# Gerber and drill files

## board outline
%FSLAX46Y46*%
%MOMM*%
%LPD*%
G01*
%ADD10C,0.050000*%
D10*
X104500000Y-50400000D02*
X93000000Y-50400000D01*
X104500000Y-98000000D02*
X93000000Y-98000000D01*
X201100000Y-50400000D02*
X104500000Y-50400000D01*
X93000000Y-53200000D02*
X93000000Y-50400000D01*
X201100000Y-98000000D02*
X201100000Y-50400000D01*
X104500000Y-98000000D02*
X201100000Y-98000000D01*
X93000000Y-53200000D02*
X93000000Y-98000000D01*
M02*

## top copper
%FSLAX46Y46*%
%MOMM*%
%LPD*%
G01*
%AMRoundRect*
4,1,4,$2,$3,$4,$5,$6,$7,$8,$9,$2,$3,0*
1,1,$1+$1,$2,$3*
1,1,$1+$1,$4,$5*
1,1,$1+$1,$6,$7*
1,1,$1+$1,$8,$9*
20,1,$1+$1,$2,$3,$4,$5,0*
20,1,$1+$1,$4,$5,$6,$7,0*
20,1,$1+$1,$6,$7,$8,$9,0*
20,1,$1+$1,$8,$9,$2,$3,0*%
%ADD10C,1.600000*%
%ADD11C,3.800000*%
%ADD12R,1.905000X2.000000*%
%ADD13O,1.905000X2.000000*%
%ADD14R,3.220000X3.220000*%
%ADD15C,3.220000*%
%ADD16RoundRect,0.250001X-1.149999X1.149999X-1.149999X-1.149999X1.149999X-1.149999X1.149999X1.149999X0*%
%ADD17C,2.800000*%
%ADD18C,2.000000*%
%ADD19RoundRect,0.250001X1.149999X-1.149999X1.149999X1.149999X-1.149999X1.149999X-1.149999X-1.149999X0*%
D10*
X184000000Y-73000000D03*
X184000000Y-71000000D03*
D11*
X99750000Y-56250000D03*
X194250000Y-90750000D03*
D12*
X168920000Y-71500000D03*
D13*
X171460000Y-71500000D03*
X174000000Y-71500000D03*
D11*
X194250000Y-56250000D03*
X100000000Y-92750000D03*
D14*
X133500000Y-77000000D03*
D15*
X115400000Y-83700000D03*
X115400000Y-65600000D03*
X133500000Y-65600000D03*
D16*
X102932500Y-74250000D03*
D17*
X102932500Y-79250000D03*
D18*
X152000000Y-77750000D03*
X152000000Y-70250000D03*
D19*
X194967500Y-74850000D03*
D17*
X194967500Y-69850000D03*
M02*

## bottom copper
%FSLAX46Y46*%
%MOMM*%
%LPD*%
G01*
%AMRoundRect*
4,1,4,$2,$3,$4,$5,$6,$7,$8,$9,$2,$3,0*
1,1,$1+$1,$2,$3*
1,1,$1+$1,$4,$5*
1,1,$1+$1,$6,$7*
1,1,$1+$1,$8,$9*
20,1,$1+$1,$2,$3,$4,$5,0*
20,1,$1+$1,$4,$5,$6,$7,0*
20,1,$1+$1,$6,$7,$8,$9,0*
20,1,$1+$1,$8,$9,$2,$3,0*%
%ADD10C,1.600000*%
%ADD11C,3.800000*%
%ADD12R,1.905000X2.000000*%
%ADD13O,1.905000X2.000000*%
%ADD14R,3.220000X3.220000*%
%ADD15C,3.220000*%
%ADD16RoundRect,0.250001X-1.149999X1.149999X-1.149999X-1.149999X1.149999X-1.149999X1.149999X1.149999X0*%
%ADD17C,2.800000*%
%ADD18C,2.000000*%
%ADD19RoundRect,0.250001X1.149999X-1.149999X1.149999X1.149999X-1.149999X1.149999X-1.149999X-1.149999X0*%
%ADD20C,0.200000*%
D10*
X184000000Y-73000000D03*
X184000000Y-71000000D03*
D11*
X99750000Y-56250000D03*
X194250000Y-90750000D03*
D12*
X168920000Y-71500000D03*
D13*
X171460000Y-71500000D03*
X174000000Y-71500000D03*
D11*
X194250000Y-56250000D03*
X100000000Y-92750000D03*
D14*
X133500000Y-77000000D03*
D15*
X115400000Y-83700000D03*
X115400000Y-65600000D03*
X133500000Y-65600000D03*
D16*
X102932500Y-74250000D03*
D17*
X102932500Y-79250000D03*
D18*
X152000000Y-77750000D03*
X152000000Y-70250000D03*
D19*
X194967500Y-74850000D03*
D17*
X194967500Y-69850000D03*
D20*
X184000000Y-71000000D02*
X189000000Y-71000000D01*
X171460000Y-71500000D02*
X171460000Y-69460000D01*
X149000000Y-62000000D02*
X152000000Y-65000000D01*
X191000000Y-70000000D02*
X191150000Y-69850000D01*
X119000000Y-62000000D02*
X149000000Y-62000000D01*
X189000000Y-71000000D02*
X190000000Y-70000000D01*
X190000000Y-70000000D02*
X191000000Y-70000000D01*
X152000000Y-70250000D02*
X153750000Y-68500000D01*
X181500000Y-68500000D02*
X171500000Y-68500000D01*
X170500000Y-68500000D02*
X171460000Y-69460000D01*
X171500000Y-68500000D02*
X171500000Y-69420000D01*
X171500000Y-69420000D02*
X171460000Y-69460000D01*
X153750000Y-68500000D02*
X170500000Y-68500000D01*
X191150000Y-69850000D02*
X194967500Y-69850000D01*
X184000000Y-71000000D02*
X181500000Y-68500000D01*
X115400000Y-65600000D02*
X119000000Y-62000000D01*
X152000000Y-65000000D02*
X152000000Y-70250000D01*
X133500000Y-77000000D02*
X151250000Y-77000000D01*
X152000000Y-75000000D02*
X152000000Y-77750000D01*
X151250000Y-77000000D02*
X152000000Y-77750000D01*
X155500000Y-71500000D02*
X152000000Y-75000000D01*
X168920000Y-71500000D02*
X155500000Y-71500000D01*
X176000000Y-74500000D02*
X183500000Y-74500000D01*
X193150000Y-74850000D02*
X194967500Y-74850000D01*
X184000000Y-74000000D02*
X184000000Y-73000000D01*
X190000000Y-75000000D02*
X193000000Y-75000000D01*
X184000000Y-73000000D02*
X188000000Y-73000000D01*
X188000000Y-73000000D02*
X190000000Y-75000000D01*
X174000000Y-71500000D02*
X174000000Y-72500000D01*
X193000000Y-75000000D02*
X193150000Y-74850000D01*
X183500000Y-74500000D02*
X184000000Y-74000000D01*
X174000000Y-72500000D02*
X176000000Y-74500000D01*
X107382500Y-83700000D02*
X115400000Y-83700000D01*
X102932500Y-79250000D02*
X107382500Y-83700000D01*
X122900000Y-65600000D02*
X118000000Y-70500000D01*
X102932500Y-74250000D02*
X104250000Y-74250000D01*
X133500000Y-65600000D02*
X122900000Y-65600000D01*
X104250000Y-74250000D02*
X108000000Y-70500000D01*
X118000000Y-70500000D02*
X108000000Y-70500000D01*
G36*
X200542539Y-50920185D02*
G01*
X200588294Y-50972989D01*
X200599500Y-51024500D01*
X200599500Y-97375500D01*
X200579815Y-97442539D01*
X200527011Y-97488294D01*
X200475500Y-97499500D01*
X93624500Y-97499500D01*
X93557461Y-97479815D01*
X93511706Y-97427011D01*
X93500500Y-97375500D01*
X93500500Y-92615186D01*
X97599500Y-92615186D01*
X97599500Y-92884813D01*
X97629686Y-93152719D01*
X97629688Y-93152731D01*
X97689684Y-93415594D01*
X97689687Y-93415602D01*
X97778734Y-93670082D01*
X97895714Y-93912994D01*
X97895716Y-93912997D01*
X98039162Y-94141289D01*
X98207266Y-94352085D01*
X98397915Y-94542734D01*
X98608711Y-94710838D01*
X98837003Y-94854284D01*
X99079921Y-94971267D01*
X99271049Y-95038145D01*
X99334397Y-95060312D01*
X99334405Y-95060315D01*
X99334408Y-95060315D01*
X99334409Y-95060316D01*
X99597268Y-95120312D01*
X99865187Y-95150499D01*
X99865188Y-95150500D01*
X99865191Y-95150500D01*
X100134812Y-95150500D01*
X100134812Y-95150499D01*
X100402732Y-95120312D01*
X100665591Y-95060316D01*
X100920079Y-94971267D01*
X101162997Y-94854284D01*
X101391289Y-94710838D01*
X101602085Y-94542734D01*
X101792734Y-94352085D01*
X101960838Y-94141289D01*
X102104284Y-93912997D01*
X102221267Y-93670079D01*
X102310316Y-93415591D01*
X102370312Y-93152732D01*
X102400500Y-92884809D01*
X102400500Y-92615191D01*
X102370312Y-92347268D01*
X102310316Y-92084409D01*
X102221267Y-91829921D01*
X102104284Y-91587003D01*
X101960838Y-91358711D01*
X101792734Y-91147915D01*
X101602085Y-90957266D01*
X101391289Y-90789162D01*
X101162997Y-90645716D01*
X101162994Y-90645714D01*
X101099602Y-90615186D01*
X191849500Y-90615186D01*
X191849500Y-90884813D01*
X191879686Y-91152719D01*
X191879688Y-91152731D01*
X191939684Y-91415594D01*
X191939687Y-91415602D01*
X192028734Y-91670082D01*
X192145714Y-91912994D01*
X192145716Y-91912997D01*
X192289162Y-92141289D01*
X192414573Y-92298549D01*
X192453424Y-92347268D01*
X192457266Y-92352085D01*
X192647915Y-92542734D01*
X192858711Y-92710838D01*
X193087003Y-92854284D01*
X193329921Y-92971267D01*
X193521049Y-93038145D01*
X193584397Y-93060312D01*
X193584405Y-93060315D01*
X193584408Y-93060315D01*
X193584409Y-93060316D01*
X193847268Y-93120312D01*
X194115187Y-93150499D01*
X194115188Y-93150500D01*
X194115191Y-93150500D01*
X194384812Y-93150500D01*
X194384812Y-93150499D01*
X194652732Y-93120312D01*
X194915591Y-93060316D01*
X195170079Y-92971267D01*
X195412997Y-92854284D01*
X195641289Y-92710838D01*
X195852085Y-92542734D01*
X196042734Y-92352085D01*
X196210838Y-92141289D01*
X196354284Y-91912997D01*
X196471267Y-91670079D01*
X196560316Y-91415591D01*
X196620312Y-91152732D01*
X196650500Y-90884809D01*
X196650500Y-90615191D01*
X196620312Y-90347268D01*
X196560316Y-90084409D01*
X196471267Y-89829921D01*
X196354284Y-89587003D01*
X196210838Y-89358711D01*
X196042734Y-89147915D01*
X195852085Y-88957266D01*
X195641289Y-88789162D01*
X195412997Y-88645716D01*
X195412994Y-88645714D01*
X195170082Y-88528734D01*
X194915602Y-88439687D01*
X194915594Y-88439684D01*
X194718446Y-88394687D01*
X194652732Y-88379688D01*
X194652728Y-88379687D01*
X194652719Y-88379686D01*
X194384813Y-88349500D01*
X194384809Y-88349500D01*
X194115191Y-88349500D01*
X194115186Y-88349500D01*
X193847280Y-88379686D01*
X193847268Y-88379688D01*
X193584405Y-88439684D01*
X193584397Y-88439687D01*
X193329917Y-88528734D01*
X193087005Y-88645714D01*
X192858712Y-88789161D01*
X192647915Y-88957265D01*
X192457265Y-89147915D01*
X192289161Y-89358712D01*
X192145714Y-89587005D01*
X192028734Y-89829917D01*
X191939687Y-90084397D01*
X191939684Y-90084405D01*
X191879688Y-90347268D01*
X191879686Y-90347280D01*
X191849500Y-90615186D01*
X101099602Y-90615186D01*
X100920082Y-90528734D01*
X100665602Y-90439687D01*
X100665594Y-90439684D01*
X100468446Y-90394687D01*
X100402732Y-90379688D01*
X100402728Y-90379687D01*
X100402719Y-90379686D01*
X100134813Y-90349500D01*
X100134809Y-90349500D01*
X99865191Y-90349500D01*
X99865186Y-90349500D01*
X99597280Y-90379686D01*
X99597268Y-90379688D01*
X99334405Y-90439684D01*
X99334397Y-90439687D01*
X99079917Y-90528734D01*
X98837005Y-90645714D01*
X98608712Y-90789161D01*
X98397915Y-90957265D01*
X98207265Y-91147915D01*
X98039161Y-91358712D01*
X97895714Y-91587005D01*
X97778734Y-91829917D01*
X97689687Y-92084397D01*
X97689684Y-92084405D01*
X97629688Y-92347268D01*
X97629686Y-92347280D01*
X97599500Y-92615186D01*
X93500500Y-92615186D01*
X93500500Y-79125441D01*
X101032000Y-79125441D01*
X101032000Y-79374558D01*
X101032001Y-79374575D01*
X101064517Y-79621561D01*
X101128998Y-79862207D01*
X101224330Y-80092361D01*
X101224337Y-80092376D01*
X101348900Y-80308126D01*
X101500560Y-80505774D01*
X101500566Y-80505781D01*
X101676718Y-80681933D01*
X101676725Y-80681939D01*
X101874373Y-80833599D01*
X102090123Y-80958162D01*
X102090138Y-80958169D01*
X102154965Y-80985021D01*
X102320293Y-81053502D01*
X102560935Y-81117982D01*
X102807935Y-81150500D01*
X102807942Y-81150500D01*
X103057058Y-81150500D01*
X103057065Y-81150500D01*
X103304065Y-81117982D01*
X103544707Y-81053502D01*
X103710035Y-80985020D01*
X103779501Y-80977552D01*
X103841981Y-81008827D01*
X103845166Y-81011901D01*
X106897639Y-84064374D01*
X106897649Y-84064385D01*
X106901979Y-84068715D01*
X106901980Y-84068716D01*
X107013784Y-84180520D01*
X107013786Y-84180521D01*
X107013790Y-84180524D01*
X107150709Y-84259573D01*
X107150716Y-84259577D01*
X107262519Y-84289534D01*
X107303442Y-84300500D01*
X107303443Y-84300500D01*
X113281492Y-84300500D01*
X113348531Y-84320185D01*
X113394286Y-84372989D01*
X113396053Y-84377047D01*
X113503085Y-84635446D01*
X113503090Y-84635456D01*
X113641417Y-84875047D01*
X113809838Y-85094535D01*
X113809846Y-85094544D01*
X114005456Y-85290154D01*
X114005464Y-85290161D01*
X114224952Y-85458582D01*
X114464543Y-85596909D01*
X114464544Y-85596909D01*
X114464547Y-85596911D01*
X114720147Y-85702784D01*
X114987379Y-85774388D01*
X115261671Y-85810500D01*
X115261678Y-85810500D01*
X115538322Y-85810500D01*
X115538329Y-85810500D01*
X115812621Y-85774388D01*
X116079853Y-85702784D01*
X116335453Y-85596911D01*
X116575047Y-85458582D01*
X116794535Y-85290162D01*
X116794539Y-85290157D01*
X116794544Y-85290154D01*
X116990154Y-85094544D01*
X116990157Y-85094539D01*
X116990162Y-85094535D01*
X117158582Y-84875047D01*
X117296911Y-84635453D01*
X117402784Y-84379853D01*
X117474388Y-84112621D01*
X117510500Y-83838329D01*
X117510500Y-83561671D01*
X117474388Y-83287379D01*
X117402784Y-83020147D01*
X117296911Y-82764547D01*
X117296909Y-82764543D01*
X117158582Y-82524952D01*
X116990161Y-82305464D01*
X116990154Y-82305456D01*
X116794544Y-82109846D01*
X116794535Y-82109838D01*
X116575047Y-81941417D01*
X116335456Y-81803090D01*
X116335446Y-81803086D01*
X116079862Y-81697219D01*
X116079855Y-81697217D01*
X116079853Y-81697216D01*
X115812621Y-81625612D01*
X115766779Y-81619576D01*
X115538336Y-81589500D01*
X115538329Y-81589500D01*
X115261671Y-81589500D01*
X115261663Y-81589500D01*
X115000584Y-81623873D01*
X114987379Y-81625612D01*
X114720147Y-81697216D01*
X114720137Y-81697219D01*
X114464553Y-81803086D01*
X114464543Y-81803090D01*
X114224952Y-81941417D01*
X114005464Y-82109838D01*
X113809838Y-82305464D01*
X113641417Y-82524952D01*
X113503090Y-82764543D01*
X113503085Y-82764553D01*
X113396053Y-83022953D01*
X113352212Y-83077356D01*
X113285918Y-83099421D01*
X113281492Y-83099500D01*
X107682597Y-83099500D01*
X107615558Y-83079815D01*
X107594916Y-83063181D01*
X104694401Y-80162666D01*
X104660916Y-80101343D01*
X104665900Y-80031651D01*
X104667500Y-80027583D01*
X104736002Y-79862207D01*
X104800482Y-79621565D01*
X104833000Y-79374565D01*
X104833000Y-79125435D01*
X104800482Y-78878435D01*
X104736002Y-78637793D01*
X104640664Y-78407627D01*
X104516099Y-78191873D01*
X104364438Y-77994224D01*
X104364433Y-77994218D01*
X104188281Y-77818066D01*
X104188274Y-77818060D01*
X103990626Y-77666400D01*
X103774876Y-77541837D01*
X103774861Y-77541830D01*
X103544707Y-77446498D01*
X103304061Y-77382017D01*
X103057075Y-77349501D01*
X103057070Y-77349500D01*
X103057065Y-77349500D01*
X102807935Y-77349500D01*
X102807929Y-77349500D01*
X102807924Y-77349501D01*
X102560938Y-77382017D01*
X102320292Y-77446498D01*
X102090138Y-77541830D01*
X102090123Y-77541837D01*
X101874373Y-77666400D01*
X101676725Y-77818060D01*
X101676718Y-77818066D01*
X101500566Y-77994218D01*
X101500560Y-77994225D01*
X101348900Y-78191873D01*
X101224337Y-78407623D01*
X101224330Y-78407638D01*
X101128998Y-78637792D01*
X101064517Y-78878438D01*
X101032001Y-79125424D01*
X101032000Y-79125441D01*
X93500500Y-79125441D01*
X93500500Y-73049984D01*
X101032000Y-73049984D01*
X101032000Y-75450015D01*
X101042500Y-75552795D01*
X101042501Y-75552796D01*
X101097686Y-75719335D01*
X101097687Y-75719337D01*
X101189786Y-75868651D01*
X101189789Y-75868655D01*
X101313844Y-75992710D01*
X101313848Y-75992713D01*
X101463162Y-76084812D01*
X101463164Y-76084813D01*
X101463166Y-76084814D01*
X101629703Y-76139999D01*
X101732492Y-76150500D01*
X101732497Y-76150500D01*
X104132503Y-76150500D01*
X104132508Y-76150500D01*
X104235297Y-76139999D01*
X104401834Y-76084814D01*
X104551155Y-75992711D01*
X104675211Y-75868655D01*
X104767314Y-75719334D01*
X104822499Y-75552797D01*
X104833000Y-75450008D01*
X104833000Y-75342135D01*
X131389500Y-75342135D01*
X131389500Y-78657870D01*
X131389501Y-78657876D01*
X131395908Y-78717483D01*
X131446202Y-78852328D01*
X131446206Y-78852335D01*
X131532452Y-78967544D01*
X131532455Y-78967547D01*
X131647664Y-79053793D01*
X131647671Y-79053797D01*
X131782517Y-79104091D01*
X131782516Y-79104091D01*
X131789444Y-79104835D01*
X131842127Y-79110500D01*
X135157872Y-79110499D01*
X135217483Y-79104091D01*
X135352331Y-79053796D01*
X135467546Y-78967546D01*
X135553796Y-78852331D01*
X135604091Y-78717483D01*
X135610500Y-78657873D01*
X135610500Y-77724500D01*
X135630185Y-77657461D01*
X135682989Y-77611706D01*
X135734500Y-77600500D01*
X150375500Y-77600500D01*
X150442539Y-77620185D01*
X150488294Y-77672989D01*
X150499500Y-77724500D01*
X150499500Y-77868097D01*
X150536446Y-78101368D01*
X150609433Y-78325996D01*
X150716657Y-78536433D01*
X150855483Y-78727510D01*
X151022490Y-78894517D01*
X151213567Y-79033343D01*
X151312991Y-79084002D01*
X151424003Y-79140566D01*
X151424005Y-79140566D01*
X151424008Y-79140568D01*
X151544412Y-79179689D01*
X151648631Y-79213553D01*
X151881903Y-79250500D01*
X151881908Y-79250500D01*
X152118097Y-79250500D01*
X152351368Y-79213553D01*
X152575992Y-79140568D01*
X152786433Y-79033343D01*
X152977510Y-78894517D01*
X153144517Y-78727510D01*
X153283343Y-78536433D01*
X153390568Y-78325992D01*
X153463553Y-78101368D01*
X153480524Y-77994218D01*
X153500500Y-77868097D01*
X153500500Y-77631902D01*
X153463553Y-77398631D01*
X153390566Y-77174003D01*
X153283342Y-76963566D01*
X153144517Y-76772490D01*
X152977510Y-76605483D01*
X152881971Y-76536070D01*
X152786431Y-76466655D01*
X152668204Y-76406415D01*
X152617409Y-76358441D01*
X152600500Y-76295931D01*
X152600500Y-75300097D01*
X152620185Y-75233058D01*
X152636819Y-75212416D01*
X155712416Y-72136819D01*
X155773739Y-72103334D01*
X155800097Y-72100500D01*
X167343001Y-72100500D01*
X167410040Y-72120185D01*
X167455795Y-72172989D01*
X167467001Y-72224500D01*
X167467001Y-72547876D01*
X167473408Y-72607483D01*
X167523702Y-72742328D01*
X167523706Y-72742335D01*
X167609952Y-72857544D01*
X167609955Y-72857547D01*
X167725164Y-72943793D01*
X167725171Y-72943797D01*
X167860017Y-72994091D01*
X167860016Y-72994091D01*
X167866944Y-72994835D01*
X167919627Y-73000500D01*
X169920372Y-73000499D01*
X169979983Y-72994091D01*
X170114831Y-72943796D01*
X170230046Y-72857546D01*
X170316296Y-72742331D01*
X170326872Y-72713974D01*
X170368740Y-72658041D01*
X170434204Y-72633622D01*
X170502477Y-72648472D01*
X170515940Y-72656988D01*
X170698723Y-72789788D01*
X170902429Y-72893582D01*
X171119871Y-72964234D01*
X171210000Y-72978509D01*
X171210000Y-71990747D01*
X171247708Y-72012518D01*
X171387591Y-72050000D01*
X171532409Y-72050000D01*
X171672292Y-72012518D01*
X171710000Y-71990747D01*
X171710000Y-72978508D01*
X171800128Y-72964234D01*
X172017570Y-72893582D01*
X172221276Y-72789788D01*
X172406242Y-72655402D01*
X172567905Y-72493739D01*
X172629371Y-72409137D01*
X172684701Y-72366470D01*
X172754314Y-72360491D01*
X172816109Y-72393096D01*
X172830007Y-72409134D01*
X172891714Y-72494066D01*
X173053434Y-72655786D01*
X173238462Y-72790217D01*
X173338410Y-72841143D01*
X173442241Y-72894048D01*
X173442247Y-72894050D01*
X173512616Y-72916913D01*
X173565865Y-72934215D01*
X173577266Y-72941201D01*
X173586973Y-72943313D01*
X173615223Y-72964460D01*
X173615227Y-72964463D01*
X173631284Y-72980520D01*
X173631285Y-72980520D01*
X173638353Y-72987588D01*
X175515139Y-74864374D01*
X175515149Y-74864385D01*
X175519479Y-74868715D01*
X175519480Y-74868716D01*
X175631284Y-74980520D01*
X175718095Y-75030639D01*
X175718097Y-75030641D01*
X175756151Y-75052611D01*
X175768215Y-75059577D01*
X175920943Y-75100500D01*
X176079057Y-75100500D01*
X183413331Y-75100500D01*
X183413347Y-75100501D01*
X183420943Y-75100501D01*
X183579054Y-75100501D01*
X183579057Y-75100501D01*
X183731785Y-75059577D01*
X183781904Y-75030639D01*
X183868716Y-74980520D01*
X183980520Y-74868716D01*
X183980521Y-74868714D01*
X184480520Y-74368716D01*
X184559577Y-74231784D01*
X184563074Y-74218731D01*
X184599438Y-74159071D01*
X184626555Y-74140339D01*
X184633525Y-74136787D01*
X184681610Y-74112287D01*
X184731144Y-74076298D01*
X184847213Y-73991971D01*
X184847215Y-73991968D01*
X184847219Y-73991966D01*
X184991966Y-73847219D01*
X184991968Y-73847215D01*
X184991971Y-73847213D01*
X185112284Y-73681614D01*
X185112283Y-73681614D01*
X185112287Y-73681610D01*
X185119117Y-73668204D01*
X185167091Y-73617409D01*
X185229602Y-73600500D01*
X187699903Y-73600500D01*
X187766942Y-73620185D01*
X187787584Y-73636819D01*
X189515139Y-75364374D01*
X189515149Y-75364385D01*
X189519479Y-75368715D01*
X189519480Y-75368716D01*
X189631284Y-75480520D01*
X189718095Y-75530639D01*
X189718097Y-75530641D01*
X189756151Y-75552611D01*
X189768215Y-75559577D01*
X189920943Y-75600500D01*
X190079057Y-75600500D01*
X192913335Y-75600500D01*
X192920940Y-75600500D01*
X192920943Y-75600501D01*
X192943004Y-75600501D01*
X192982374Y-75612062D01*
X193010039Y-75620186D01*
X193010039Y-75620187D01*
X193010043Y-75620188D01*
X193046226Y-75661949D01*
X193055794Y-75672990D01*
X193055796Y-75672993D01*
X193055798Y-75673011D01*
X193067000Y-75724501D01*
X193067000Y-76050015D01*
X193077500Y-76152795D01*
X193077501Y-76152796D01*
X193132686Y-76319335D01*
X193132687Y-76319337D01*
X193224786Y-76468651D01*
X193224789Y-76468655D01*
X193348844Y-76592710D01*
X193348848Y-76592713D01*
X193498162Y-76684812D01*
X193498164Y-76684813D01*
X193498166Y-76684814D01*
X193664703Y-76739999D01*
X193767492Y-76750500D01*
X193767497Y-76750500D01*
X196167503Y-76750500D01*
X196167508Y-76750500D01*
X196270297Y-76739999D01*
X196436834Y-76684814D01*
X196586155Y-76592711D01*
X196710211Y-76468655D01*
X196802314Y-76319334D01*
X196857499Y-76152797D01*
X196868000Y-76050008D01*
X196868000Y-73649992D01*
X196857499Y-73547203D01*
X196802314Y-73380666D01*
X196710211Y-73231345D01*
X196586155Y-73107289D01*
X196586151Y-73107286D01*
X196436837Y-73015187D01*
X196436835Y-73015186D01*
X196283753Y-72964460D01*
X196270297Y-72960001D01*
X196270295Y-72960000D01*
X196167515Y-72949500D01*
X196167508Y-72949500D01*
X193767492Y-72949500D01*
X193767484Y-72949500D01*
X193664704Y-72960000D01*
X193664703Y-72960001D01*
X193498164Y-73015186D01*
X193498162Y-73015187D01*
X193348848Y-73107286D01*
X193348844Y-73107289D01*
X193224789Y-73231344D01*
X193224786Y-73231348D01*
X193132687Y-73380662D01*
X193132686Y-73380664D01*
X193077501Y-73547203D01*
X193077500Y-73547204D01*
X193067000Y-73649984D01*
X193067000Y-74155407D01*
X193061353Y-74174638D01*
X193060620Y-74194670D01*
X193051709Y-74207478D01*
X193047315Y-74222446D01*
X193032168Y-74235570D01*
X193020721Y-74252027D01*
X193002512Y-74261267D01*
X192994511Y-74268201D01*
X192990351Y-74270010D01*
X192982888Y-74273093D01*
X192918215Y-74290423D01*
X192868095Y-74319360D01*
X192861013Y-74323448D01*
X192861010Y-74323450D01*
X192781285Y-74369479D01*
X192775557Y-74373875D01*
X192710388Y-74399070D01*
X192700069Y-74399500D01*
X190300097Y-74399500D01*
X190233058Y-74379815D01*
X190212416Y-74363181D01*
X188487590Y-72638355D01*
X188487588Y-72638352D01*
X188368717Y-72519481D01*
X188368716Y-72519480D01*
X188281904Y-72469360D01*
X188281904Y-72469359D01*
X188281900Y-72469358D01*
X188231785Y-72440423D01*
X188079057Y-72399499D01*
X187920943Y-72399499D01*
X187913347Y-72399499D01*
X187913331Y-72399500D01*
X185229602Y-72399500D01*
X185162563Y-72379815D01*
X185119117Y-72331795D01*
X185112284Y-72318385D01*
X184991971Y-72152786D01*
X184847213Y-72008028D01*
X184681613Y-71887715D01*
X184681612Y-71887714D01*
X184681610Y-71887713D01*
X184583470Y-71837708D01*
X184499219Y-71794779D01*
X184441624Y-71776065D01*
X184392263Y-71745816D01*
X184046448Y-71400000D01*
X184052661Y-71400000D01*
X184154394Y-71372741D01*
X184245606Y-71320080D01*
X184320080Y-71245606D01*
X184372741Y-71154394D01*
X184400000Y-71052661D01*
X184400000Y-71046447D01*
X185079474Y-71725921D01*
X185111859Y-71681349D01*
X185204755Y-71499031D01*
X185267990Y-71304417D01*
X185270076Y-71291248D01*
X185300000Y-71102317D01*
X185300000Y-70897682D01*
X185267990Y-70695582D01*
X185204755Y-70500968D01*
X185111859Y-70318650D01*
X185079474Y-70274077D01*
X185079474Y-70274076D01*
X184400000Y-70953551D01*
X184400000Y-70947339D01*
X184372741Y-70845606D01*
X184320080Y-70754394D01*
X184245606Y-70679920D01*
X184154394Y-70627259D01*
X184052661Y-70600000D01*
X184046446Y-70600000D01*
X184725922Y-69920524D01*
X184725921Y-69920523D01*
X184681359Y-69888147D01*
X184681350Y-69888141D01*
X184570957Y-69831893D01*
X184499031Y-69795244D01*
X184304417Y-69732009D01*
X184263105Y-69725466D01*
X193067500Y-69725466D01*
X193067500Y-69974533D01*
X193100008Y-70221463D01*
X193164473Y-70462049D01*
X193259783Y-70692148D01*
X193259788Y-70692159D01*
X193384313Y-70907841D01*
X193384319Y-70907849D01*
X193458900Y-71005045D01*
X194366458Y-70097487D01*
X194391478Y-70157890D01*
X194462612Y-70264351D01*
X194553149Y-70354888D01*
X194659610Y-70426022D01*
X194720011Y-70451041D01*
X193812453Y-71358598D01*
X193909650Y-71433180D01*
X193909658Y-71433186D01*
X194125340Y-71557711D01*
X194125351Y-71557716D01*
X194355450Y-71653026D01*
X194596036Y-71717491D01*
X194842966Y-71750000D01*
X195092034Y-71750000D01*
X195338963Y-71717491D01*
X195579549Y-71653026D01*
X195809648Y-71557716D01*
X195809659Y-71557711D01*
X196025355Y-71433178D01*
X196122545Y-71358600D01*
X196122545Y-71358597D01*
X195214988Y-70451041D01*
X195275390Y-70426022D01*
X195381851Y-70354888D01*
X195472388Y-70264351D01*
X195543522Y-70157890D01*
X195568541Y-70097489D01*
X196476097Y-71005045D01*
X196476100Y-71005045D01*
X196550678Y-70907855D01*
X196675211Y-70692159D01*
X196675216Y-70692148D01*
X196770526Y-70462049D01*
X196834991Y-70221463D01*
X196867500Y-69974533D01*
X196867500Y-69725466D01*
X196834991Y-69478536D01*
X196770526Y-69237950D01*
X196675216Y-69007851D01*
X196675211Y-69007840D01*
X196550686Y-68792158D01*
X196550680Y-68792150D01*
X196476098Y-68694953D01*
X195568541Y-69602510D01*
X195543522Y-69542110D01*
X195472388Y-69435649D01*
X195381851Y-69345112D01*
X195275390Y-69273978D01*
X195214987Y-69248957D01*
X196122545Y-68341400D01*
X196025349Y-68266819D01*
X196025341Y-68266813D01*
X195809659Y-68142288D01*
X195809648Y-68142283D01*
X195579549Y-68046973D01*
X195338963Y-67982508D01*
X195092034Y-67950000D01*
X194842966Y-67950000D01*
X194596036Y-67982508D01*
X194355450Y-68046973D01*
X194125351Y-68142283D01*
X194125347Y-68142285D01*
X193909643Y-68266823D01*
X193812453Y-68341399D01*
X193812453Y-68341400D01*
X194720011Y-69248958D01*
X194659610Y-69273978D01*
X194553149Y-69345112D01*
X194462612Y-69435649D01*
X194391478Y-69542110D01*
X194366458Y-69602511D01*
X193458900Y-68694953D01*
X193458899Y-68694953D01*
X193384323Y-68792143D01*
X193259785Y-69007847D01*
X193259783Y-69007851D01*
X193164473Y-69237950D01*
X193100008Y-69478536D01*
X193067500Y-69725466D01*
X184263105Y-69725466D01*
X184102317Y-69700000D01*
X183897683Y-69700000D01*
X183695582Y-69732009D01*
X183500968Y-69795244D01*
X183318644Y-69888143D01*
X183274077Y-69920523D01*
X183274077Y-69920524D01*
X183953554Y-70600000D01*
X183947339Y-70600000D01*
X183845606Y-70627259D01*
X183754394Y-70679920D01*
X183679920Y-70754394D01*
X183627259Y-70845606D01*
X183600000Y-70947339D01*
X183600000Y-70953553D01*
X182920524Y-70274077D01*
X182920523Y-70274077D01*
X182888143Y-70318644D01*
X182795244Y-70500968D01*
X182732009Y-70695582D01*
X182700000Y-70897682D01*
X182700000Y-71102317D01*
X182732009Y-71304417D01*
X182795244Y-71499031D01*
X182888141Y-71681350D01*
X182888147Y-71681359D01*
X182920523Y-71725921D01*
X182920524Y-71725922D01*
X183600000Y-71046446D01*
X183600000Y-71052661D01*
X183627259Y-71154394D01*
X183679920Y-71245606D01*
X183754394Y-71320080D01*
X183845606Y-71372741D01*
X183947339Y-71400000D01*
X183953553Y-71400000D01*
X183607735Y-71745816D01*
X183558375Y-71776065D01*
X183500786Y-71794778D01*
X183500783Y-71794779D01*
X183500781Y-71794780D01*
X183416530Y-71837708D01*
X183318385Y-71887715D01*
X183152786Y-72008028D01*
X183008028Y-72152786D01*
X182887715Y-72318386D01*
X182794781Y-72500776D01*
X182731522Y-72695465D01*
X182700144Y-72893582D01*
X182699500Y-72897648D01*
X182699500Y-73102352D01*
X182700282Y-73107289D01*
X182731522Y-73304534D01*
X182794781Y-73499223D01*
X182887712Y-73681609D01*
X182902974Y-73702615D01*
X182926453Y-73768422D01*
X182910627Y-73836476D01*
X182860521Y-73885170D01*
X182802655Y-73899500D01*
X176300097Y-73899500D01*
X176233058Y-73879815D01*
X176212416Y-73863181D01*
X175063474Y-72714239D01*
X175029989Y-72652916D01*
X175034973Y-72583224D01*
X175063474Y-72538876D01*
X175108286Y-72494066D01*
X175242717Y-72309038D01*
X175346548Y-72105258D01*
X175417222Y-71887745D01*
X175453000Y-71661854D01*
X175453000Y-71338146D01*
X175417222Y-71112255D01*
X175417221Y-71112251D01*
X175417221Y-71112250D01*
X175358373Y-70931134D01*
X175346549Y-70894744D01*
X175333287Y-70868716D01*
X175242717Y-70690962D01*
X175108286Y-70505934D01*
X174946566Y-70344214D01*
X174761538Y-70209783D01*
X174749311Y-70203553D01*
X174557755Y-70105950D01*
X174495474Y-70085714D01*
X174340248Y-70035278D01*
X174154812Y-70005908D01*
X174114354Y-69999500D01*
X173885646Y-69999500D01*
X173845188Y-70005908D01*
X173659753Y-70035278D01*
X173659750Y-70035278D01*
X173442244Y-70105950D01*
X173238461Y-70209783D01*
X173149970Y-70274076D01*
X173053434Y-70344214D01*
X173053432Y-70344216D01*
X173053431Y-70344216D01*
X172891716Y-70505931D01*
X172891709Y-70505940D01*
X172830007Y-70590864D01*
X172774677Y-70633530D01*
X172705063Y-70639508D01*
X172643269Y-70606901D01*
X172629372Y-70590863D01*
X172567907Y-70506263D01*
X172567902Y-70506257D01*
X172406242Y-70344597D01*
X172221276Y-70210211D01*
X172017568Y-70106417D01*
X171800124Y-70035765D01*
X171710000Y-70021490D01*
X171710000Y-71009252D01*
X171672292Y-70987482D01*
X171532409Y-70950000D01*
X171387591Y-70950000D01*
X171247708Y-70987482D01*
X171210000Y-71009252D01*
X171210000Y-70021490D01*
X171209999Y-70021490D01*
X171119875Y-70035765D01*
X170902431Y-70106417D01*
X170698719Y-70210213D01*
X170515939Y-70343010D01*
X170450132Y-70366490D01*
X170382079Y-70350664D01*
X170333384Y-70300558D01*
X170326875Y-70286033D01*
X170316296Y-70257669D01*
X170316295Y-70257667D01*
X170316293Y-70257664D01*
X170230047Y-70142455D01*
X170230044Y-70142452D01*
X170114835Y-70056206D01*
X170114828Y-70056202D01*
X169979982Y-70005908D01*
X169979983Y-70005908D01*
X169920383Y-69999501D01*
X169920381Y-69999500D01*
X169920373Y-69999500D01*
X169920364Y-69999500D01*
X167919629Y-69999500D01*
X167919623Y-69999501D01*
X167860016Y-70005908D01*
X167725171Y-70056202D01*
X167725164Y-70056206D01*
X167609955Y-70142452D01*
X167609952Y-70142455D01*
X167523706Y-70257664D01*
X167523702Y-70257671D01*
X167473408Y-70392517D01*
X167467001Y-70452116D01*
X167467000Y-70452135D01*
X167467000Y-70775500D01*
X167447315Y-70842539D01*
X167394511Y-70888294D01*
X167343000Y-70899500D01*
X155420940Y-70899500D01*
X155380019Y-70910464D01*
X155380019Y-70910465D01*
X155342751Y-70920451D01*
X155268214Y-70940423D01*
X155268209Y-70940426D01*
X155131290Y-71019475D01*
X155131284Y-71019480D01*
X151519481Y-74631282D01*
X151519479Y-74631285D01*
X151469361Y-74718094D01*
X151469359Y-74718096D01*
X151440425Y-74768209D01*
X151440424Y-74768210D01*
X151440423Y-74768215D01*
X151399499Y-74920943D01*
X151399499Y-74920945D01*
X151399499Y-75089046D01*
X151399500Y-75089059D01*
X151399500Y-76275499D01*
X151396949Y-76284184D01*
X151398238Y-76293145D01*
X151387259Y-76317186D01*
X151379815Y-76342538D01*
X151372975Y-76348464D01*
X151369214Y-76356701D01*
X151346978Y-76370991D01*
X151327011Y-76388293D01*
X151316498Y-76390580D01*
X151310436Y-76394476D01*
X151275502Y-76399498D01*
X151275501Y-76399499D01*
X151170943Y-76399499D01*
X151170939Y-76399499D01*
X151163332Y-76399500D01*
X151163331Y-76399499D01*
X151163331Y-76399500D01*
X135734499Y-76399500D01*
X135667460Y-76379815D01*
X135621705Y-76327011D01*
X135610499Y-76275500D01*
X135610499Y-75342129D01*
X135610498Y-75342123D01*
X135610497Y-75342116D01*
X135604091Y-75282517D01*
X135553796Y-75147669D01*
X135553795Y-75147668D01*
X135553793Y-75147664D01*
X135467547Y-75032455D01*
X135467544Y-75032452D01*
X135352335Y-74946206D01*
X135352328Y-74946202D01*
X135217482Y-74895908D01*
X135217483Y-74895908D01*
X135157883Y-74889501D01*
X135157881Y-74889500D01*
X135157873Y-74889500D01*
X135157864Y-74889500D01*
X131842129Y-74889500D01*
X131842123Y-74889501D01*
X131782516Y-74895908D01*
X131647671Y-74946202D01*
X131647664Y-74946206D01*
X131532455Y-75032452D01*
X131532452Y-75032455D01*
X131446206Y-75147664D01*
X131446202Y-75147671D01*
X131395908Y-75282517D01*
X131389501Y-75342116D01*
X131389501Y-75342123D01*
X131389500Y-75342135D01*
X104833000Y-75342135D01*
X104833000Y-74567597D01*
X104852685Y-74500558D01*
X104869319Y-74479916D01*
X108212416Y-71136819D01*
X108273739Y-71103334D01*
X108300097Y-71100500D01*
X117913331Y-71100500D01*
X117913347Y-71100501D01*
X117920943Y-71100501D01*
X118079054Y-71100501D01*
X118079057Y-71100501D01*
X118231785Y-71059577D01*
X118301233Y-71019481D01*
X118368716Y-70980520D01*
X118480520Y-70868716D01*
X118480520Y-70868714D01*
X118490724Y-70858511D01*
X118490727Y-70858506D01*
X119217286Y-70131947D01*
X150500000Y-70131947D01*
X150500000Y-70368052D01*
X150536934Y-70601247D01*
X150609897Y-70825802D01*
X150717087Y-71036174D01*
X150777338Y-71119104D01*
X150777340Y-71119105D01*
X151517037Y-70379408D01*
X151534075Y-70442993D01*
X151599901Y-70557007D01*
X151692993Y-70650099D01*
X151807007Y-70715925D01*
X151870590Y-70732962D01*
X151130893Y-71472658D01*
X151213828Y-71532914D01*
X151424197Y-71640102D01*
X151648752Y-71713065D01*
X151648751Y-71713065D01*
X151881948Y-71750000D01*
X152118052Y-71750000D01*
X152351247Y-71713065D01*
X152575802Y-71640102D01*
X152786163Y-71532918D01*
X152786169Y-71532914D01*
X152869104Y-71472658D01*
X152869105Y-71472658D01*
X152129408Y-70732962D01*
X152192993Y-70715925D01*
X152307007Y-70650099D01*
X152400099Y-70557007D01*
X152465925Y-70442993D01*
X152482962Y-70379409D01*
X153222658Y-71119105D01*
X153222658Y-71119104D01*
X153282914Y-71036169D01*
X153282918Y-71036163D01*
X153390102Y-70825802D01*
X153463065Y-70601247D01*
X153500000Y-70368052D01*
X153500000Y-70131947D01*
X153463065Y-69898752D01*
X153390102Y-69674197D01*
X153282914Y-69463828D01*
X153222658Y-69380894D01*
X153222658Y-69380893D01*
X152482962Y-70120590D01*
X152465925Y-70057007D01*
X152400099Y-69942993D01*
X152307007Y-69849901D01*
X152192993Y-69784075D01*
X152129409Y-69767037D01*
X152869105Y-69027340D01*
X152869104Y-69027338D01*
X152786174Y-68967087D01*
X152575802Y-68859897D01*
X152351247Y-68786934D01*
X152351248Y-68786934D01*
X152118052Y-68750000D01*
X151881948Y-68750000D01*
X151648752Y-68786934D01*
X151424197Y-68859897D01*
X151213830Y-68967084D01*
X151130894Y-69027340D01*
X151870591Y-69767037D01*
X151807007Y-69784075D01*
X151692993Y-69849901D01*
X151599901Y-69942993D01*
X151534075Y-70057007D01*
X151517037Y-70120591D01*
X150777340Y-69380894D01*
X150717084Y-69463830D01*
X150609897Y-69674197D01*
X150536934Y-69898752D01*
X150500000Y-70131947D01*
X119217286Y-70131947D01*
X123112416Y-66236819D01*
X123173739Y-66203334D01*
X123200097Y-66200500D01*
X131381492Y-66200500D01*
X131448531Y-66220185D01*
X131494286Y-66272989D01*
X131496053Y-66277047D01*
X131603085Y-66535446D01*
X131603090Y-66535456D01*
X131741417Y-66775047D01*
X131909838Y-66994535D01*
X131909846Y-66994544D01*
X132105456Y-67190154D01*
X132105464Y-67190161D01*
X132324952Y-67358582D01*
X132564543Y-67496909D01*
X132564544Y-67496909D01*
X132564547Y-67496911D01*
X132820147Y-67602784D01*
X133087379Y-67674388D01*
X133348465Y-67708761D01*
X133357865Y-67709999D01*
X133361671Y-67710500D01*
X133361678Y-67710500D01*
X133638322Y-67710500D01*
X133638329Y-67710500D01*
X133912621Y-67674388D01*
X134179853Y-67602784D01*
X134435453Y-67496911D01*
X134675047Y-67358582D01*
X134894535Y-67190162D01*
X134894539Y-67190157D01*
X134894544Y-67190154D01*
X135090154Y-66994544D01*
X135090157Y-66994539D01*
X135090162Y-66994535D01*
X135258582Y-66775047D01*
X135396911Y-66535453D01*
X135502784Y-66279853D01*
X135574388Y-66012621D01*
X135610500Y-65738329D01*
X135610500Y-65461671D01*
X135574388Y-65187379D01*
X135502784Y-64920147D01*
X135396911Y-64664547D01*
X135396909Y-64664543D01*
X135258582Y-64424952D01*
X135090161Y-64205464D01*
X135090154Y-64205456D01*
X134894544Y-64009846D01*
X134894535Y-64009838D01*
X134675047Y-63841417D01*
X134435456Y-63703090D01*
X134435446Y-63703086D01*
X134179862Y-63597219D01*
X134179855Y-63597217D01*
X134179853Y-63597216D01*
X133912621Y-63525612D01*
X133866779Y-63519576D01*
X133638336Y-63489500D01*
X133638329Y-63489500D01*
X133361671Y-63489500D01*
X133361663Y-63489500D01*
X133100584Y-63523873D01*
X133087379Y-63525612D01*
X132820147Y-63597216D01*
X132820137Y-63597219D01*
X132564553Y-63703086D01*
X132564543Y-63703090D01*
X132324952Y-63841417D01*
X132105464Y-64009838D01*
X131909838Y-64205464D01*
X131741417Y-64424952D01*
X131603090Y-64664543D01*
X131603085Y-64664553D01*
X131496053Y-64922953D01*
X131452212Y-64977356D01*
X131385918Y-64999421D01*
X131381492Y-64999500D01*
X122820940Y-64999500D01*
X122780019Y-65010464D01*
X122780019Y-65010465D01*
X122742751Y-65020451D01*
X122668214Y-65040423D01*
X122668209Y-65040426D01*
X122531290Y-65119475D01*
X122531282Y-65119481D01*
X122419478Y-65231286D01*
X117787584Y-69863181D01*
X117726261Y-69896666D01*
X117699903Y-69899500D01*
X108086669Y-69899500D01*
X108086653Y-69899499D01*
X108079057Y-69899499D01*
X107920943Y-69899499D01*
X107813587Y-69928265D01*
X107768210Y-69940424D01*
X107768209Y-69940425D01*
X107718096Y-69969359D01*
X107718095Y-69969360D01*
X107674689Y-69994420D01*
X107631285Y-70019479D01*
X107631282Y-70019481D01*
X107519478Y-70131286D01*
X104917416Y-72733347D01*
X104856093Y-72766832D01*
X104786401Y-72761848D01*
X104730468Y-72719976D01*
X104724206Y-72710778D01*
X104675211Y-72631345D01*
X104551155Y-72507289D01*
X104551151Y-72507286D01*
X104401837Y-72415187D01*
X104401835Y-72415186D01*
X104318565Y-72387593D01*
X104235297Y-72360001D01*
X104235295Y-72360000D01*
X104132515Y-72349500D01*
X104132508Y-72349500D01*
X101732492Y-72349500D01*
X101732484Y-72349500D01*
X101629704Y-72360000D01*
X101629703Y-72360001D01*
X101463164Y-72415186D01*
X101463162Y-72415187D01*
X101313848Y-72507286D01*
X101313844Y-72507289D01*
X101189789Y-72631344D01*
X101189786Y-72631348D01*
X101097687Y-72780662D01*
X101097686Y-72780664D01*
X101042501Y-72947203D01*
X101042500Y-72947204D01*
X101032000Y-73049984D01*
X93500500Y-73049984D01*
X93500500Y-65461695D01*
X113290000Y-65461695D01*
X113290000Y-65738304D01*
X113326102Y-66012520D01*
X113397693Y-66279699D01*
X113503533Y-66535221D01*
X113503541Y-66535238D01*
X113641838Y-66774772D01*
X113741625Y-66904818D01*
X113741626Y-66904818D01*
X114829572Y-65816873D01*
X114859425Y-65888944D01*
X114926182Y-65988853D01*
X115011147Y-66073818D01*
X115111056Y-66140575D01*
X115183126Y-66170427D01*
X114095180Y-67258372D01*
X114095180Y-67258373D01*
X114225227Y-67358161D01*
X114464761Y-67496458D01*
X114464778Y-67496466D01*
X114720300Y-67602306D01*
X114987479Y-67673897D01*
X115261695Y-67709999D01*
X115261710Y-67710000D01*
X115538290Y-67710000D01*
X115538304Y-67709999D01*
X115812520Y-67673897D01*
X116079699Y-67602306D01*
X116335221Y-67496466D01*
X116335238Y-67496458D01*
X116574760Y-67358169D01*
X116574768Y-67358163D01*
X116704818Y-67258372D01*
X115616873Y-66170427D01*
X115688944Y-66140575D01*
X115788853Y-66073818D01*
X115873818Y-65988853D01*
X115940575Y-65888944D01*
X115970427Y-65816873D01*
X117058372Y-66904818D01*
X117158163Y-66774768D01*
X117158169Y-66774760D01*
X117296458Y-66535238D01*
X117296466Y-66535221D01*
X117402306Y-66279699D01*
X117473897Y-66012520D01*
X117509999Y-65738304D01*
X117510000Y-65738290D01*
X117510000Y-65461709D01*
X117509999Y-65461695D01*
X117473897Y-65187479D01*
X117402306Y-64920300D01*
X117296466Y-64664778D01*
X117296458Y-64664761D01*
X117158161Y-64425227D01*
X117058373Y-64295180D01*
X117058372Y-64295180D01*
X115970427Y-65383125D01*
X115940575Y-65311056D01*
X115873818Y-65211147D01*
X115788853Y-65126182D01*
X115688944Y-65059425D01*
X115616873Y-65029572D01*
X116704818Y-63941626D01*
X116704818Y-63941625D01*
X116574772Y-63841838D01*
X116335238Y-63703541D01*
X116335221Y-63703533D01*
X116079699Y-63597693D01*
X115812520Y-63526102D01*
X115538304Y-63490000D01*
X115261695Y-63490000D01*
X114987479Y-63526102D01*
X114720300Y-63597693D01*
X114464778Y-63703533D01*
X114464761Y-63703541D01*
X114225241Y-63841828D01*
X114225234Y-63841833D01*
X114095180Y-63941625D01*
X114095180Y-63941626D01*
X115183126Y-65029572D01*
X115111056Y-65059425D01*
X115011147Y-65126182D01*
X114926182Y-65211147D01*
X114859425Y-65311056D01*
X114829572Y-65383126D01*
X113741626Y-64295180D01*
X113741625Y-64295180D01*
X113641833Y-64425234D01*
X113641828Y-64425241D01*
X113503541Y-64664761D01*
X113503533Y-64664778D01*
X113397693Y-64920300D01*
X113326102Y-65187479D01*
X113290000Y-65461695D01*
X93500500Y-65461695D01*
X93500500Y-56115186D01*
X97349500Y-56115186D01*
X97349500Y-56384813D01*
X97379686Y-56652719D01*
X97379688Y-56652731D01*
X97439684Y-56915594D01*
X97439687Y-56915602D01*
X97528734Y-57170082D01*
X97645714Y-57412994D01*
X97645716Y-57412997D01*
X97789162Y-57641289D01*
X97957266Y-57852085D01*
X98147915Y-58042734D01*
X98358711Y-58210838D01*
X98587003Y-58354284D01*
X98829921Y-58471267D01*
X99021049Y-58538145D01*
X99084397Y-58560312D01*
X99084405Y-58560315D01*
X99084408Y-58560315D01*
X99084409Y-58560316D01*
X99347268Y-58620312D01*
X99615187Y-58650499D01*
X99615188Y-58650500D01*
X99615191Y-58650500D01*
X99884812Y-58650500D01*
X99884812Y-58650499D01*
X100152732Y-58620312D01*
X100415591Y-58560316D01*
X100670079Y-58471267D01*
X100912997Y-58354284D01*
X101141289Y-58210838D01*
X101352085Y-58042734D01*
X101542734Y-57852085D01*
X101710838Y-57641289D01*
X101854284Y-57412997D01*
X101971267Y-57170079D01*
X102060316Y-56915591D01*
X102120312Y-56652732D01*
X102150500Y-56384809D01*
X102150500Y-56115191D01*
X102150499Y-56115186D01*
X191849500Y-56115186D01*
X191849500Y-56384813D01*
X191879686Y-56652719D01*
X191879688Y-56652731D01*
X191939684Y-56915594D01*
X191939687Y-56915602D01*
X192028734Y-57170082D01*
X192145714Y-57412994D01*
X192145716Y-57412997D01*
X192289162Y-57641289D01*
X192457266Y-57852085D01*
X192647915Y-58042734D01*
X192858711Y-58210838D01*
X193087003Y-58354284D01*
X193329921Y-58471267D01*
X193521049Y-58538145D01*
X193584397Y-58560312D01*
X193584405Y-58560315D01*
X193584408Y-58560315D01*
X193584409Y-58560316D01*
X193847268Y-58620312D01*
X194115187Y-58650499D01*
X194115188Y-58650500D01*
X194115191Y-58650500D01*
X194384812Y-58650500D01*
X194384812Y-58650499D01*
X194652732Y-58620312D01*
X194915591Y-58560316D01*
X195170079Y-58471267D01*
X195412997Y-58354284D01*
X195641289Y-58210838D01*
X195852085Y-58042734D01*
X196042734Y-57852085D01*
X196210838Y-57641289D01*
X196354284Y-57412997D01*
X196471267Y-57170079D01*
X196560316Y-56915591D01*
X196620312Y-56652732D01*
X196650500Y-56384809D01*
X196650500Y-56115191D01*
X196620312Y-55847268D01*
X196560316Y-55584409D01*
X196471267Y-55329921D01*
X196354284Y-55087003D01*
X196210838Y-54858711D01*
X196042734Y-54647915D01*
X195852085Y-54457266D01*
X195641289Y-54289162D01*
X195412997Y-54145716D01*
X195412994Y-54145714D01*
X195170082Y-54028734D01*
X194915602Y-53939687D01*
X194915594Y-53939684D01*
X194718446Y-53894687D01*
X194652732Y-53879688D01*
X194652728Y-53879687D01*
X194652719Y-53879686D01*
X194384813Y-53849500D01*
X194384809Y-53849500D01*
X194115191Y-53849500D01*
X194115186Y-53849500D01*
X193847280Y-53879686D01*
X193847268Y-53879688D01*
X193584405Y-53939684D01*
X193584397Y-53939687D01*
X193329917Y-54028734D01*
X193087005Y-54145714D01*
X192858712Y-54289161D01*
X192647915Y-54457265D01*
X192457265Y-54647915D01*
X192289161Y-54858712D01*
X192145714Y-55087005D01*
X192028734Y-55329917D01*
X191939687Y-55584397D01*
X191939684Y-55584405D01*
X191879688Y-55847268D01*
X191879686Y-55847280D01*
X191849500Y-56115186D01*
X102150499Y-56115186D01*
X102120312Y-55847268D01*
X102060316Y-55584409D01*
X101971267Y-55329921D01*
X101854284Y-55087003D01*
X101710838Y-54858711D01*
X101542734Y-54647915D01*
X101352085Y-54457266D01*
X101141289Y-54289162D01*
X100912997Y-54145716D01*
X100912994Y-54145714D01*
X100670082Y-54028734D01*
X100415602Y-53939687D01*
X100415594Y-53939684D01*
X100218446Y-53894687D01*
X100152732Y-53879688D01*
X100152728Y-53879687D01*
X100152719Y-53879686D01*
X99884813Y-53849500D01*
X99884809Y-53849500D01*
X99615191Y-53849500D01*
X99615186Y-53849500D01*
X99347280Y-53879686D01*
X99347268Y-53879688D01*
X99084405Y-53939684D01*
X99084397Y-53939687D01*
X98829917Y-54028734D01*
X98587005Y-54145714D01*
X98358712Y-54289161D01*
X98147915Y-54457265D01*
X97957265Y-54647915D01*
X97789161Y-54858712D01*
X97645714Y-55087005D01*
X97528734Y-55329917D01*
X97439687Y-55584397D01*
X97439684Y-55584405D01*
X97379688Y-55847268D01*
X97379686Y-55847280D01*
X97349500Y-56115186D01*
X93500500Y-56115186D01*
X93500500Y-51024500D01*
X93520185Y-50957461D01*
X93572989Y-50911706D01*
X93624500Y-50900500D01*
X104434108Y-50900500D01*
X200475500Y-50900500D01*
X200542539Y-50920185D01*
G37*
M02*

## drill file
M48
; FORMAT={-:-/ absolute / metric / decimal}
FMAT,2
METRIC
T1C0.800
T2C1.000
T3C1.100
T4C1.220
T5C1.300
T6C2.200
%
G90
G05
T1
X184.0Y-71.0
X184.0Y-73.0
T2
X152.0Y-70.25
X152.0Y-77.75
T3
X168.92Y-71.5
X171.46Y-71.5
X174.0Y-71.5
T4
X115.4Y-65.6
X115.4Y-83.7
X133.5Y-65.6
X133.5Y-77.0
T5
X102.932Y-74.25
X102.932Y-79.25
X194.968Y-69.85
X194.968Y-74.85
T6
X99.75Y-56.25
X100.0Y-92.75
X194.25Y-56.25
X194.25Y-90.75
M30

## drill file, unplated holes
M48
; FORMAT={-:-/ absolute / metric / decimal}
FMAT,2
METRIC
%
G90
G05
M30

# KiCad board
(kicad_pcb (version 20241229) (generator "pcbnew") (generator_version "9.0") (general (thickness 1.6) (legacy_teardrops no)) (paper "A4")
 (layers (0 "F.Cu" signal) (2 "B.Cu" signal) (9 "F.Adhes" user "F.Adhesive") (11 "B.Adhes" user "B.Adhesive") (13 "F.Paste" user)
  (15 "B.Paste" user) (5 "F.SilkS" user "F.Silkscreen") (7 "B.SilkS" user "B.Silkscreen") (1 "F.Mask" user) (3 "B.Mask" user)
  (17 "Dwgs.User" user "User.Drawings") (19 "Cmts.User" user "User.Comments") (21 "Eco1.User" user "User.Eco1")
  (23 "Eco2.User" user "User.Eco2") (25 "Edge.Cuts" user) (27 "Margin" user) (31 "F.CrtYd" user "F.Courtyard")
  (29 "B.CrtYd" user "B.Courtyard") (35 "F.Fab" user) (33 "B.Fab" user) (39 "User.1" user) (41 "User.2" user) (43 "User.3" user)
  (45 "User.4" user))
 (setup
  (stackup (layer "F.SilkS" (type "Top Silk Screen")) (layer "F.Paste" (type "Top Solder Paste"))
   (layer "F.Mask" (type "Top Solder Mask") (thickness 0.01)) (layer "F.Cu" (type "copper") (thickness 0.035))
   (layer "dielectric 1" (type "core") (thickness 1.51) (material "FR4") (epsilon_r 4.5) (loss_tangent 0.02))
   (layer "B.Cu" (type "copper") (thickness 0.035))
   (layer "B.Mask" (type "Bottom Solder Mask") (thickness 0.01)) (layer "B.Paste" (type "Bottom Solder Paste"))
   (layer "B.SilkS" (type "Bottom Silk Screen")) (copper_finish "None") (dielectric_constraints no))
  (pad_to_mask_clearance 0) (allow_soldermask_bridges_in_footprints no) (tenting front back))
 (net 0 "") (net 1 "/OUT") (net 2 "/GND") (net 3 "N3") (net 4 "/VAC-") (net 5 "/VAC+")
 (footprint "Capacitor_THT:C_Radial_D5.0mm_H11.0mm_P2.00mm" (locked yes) (layer "F.Cu") (at 184 73 90)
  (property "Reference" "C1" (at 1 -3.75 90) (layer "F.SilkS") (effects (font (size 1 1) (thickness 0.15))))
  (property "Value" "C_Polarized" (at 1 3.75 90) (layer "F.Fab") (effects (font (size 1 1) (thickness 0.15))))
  (pad "1" thru_hole circle (at 0 0 90) (size 1.6 1.6) (drill 0.8) (layers "*.Cu" "*.Mask") (remove_unused_layers no) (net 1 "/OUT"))
  (pad "2" thru_hole circle (at 2 0 90) (size 1.6 1.6) (drill 0.8) (layers "*.Cu" "*.Mask") (remove_unused_layers no) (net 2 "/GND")))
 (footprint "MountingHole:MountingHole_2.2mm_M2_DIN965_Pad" (layer "F.Cu") (at 99.75 56.25)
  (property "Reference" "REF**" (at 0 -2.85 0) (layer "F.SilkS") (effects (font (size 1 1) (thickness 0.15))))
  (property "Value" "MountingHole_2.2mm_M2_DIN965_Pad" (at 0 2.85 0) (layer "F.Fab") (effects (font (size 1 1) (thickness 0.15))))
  (pad "1" thru_hole circle (at 0 0) (size 3.8 3.8) (drill 2.2) (layers "*.Cu" "*.Mask") (remove_unused_layers no) (zone_connect 2)))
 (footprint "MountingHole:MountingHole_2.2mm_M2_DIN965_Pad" (layer "F.Cu") (at 194.25 90.75)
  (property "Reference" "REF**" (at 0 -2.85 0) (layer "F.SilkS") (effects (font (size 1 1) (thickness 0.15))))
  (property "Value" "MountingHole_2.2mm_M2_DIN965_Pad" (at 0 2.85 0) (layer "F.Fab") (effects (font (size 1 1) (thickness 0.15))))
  (pad "1" thru_hole circle (at 0 0) (size 3.8 3.8) (drill 2.2) (layers "*.Cu" "*.Mask") (remove_unused_layers no) (zone_connect 2)))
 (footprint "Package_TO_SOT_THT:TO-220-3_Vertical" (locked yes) (layer "F.Cu") (at 168.92 71.5)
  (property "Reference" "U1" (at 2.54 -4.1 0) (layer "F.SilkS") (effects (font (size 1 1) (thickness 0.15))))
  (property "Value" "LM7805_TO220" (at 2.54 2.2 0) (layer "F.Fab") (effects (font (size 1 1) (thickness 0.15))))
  (pad "1" thru_hole rect (at 0 0) (size 1.905 2) (drill 1.1) (layers "*.Cu" "*.Mask") (remove_unused_layers no) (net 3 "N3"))
  (pad "2" thru_hole oval (at 2.54 0) (size 1.905 2) (drill 1.1) (layers "*.Cu" "*.Mask") (remove_unused_layers no) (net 2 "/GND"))
  (pad "3" thru_hole oval (at 5.08 0) (size 1.905 2) (drill 1.1) (layers "*.Cu" "*.Mask") (remove_unused_layers no) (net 1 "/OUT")))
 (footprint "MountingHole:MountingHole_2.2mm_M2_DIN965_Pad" (layer "F.Cu") (at 194.25 56.25)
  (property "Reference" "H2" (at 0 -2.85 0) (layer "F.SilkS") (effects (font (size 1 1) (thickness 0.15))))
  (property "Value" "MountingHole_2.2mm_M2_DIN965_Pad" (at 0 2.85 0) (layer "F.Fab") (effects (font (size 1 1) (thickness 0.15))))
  (pad "1" thru_hole circle (at 0 0) (size 3.8 3.8) (drill 2.2) (layers "*.Cu" "*.Mask") (remove_unused_layers no) (zone_connect 2)))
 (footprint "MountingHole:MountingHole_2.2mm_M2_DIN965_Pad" (layer "F.Cu") (at 100 92.75)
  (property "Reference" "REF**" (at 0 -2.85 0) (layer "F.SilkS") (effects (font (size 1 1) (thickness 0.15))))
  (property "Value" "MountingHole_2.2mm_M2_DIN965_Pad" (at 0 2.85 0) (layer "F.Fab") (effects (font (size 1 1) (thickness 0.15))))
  (pad "1" thru_hole circle (at 0 0) (size 3.8 3.8) (drill 2.2) (layers "*.Cu" "*.Mask") (remove_unused_layers no) (zone_connect 2)))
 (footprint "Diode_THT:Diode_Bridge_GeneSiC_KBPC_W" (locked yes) (layer "F.Cu") (at 133.5 77 180)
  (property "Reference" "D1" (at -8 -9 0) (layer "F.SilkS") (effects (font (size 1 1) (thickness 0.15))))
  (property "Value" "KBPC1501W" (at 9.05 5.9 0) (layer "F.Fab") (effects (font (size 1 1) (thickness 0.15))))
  (pad "1" thru_hole rect (at 0 0) (size 3.22 3.22) (drill 1.22) (layers "*.Cu" "*.Mask") (remove_unused_layers no) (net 3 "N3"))
  (pad "2" thru_hole circle (at 18.1 -6.7) (size 3.22 3.22) (drill 1.22) (layers "*.Cu" "*.Mask") (remove_unused_layers no) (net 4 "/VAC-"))
  (pad "3" thru_hole circle (at 18.1 11.4 90) (size 3.22 3.22) (drill 1.22) (layers "*.Cu" "*.Mask") (remove_unused_layers no)
   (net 2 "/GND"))
  (pad "4" thru_hole circle (at 0 11.4) (size 3.22 3.22) (drill 1.22) (layers "*.Cu" "*.Mask") (remove_unused_layers no) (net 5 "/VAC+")))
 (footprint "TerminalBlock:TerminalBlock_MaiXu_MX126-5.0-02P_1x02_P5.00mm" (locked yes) (layer "F.Cu") (at 102.9325 74.25 -90)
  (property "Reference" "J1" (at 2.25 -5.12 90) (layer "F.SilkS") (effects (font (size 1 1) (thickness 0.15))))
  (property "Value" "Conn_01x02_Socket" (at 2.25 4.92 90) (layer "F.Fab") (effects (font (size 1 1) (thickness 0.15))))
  (pad "1" thru_hole roundrect (at 0 0 270) (size 2.8 2.8) (drill 1.3) (layers "*.Cu" "*.Mask") (remove_unused_layers no)
   (roundrect_rratio 0.089286) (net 5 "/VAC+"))
  (pad "2" thru_hole circle (at 5 0 270) (size 2.8 2.8) (drill 1.3) (layers "*.Cu" "*.Mask") (remove_unused_layers no) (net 4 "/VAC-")))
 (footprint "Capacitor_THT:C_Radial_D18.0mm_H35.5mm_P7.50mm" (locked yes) (layer "F.Cu") (at 152 77.75 90)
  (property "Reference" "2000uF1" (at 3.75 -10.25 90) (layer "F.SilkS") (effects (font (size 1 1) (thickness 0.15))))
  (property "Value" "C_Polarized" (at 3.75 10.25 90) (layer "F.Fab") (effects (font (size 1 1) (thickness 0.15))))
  (pad "1" thru_hole circle (at 0 0 90) (size 2 2) (drill 1) (layers "*.Cu" "*.Mask") (remove_unused_layers no) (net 3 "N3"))
  (pad "2" thru_hole circle (at 7.5 0 90) (size 2 2) (drill 1) (layers "*.Cu" "*.Mask") (remove_unused_layers no) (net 2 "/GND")))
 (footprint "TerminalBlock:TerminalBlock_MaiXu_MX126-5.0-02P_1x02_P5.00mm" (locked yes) (layer "F.Cu") (at 194.9675 74.85 90)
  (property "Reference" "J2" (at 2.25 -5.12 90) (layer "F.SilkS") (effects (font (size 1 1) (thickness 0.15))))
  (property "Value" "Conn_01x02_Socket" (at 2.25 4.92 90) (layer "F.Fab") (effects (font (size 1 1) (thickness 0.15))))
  (pad "1" thru_hole roundrect (at 0 0 90) (size 2.8 2.8) (drill 1.3) (layers "*.Cu" "*.Mask") (remove_unused_layers no)
   (roundrect_rratio 0.089286) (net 1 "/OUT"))
  (pad "2" thru_hole circle (at 5 0 90) (size 2.8 2.8) (drill 1.3) (layers "*.Cu" "*.Mask") (remove_unused_layers no) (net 2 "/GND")))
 (gr_line (start 104.5 50.4) (end 93 50.4) (stroke (width 0.05) (type default)) (locked yes) (layer "Edge.Cuts"))
 (gr_line (start 104.5 98) (end 93 98) (stroke (width 0.05) (type default)) (locked yes) (layer "Edge.Cuts"))
 (gr_line (start 201.1 50.4) (end 104.5 50.4) (stroke (width 0.05) (type default)) (locked yes) (layer "Edge.Cuts"))
 (gr_line (start 93 53.2) (end 93 50.4) (stroke (width 0.05) (type default)) (locked yes) (layer "Edge.Cuts"))
 (gr_line (start 201.1 98) (end 201.1 50.4) (stroke (width 0.05) (type default)) (locked yes) (layer "Edge.Cuts"))
 (gr_line (start 104.5 98) (end 201.1 98) (stroke (width 0.05) (type default)) (locked yes) (layer "Edge.Cuts"))
 (gr_line (start 93 53.2) (end 93 98) (stroke (width 0.05) (type default)) (locked yes) (layer "Edge.Cuts"))
 (segment (start 184 71) (end 189 71) (width 0.2) (locked yes) (layer "B.Cu") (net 2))
 (segment (start 171.46 71.5) (end 171.46 69.46) (width 0.2) (locked yes) (layer "B.Cu") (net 2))
 (segment (start 149 62) (end 152 65) (width 0.2) (locked yes) (layer "B.Cu") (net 2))
 (segment (start 191 70) (end 191.15 69.85) (width 0.2) (locked yes) (layer "B.Cu") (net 2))
 (segment (start 119 62) (end 149 62) (width 0.2) (locked yes) (layer "B.Cu") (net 2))
 (segment (start 189 71) (end 190 70) (width 0.2) (locked yes) (layer "B.Cu") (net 2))
 (segment (start 190 70) (end 191 70) (width 0.2) (locked yes) (layer "B.Cu") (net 2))
 (segment (start 152 70.25) (end 153.75 68.5) (width 0.2) (locked yes) (layer "B.Cu") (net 2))
 (segment (start 181.5 68.5) (end 171.5 68.5) (width 0.2) (locked yes) (layer "B.Cu") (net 2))
 (segment (start 170.5 68.5) (end 171.46 69.46) (width 0.2) (locked yes) (layer "B.Cu") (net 2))
 (segment (start 171.5 68.5) (end 171.5 69.42) (width 0.2) (locked yes) (layer "B.Cu") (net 2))
 (segment (start 171.5 69.42) (end 171.46 69.46) (width 0.2) (locked yes) (layer "B.Cu") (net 2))
 (segment (start 153.75 68.5) (end 170.5 68.5) (width 0.2) (locked yes) (layer "B.Cu") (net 2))
 (segment (start 191.15 69.85) (end 194.9675 69.85) (width 0.2) (locked yes) (layer "B.Cu") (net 2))
 (segment (start 184 71) (end 181.5 68.5) (width 0.2) (locked yes) (layer "B.Cu") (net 2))
 (segment (start 115.4 65.6) (end 119 62) (width 0.2) (locked yes) (layer "B.Cu") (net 2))
 (segment (start 152 65) (end 152 70.25) (width 0.2) (locked yes) (layer "B.Cu") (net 2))
 (segment (start 133.5 77) (end 151.25 77) (width 0.2) (locked yes) (layer "B.Cu") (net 3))
 (segment (start 152 75) (end 152 77.75) (width 0.2) (locked yes) (layer "B.Cu") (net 3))
 (segment (start 151.25 77) (end 152 77.75) (width 0.2) (locked yes) (layer "B.Cu") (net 3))
 (segment (start 155.5 71.5) (end 152 75) (width 0.2) (locked yes) (layer "B.Cu") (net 3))
 (segment (start 168.92 71.5) (end 155.5 71.5) (width 0.2) (locked yes) (layer "B.Cu") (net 3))
 (segment (start 176 74.5) (end 183.5 74.5) (width 0.2) (locked yes) (layer "B.Cu") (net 1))
 (segment (start 193.15 74.85) (end 194.9675 74.85) (width 0.2) (locked yes) (layer "B.Cu") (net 1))
 (segment (start 184 74) (end 184 73) (width 0.2) (locked yes) (layer "B.Cu") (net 1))
 (segment (start 190 75) (end 193 75) (width 0.2) (locked yes) (layer "B.Cu") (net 1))
 (segment (start 184 73) (end 188 73) (width 0.2) (locked yes) (layer "B.Cu") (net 1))
 (segment (start 188 73) (end 190 75) (width 0.2) (locked yes) (layer "B.Cu") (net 1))
 (segment (start 174 71.5) (end 174 72.5) (width 0.2) (locked yes) (layer "B.Cu") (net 1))
 (segment (start 193 75) (end 193.15 74.85) (width 0.2) (locked yes) (layer "B.Cu") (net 1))
 (segment (start 183.5 74.5) (end 184 74) (width 0.2) (locked yes) (layer "B.Cu") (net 1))
 (segment (start 174 72.5) (end 176 74.5) (width 0.2) (locked yes) (layer "B.Cu") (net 1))
 (segment (start 107.3825 83.7) (end 115.4 83.7) (width 0.2) (locked yes) (layer "B.Cu") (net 4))
 (segment (start 102.9325 79.25) (end 107.3825 83.7) (width 0.2) (locked yes) (layer "B.Cu") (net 4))
 (segment (start 122.9 65.6) (end 118 70.5) (width 0.2) (locked yes) (layer "B.Cu") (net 5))
 (segment (start 102.9325 74.25) (end 104.25 74.25) (width 0.2) (locked yes) (layer "B.Cu") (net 5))
 (segment (start 133.5 65.6) (end 122.9 65.6) (width 0.2) (locked yes) (layer "B.Cu") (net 5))
 (segment (start 104.25 74.25) (end 108 70.5) (width 0.2) (locked yes) (layer "B.Cu") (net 5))
 (segment (start 118 70.5) (end 108 70.5) (width 0.2) (locked yes) (layer "B.Cu") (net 5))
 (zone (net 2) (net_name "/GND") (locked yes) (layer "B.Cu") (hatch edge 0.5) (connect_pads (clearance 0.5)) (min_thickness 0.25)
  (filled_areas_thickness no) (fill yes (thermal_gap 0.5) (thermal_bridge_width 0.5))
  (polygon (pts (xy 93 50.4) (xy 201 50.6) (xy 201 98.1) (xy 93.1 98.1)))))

